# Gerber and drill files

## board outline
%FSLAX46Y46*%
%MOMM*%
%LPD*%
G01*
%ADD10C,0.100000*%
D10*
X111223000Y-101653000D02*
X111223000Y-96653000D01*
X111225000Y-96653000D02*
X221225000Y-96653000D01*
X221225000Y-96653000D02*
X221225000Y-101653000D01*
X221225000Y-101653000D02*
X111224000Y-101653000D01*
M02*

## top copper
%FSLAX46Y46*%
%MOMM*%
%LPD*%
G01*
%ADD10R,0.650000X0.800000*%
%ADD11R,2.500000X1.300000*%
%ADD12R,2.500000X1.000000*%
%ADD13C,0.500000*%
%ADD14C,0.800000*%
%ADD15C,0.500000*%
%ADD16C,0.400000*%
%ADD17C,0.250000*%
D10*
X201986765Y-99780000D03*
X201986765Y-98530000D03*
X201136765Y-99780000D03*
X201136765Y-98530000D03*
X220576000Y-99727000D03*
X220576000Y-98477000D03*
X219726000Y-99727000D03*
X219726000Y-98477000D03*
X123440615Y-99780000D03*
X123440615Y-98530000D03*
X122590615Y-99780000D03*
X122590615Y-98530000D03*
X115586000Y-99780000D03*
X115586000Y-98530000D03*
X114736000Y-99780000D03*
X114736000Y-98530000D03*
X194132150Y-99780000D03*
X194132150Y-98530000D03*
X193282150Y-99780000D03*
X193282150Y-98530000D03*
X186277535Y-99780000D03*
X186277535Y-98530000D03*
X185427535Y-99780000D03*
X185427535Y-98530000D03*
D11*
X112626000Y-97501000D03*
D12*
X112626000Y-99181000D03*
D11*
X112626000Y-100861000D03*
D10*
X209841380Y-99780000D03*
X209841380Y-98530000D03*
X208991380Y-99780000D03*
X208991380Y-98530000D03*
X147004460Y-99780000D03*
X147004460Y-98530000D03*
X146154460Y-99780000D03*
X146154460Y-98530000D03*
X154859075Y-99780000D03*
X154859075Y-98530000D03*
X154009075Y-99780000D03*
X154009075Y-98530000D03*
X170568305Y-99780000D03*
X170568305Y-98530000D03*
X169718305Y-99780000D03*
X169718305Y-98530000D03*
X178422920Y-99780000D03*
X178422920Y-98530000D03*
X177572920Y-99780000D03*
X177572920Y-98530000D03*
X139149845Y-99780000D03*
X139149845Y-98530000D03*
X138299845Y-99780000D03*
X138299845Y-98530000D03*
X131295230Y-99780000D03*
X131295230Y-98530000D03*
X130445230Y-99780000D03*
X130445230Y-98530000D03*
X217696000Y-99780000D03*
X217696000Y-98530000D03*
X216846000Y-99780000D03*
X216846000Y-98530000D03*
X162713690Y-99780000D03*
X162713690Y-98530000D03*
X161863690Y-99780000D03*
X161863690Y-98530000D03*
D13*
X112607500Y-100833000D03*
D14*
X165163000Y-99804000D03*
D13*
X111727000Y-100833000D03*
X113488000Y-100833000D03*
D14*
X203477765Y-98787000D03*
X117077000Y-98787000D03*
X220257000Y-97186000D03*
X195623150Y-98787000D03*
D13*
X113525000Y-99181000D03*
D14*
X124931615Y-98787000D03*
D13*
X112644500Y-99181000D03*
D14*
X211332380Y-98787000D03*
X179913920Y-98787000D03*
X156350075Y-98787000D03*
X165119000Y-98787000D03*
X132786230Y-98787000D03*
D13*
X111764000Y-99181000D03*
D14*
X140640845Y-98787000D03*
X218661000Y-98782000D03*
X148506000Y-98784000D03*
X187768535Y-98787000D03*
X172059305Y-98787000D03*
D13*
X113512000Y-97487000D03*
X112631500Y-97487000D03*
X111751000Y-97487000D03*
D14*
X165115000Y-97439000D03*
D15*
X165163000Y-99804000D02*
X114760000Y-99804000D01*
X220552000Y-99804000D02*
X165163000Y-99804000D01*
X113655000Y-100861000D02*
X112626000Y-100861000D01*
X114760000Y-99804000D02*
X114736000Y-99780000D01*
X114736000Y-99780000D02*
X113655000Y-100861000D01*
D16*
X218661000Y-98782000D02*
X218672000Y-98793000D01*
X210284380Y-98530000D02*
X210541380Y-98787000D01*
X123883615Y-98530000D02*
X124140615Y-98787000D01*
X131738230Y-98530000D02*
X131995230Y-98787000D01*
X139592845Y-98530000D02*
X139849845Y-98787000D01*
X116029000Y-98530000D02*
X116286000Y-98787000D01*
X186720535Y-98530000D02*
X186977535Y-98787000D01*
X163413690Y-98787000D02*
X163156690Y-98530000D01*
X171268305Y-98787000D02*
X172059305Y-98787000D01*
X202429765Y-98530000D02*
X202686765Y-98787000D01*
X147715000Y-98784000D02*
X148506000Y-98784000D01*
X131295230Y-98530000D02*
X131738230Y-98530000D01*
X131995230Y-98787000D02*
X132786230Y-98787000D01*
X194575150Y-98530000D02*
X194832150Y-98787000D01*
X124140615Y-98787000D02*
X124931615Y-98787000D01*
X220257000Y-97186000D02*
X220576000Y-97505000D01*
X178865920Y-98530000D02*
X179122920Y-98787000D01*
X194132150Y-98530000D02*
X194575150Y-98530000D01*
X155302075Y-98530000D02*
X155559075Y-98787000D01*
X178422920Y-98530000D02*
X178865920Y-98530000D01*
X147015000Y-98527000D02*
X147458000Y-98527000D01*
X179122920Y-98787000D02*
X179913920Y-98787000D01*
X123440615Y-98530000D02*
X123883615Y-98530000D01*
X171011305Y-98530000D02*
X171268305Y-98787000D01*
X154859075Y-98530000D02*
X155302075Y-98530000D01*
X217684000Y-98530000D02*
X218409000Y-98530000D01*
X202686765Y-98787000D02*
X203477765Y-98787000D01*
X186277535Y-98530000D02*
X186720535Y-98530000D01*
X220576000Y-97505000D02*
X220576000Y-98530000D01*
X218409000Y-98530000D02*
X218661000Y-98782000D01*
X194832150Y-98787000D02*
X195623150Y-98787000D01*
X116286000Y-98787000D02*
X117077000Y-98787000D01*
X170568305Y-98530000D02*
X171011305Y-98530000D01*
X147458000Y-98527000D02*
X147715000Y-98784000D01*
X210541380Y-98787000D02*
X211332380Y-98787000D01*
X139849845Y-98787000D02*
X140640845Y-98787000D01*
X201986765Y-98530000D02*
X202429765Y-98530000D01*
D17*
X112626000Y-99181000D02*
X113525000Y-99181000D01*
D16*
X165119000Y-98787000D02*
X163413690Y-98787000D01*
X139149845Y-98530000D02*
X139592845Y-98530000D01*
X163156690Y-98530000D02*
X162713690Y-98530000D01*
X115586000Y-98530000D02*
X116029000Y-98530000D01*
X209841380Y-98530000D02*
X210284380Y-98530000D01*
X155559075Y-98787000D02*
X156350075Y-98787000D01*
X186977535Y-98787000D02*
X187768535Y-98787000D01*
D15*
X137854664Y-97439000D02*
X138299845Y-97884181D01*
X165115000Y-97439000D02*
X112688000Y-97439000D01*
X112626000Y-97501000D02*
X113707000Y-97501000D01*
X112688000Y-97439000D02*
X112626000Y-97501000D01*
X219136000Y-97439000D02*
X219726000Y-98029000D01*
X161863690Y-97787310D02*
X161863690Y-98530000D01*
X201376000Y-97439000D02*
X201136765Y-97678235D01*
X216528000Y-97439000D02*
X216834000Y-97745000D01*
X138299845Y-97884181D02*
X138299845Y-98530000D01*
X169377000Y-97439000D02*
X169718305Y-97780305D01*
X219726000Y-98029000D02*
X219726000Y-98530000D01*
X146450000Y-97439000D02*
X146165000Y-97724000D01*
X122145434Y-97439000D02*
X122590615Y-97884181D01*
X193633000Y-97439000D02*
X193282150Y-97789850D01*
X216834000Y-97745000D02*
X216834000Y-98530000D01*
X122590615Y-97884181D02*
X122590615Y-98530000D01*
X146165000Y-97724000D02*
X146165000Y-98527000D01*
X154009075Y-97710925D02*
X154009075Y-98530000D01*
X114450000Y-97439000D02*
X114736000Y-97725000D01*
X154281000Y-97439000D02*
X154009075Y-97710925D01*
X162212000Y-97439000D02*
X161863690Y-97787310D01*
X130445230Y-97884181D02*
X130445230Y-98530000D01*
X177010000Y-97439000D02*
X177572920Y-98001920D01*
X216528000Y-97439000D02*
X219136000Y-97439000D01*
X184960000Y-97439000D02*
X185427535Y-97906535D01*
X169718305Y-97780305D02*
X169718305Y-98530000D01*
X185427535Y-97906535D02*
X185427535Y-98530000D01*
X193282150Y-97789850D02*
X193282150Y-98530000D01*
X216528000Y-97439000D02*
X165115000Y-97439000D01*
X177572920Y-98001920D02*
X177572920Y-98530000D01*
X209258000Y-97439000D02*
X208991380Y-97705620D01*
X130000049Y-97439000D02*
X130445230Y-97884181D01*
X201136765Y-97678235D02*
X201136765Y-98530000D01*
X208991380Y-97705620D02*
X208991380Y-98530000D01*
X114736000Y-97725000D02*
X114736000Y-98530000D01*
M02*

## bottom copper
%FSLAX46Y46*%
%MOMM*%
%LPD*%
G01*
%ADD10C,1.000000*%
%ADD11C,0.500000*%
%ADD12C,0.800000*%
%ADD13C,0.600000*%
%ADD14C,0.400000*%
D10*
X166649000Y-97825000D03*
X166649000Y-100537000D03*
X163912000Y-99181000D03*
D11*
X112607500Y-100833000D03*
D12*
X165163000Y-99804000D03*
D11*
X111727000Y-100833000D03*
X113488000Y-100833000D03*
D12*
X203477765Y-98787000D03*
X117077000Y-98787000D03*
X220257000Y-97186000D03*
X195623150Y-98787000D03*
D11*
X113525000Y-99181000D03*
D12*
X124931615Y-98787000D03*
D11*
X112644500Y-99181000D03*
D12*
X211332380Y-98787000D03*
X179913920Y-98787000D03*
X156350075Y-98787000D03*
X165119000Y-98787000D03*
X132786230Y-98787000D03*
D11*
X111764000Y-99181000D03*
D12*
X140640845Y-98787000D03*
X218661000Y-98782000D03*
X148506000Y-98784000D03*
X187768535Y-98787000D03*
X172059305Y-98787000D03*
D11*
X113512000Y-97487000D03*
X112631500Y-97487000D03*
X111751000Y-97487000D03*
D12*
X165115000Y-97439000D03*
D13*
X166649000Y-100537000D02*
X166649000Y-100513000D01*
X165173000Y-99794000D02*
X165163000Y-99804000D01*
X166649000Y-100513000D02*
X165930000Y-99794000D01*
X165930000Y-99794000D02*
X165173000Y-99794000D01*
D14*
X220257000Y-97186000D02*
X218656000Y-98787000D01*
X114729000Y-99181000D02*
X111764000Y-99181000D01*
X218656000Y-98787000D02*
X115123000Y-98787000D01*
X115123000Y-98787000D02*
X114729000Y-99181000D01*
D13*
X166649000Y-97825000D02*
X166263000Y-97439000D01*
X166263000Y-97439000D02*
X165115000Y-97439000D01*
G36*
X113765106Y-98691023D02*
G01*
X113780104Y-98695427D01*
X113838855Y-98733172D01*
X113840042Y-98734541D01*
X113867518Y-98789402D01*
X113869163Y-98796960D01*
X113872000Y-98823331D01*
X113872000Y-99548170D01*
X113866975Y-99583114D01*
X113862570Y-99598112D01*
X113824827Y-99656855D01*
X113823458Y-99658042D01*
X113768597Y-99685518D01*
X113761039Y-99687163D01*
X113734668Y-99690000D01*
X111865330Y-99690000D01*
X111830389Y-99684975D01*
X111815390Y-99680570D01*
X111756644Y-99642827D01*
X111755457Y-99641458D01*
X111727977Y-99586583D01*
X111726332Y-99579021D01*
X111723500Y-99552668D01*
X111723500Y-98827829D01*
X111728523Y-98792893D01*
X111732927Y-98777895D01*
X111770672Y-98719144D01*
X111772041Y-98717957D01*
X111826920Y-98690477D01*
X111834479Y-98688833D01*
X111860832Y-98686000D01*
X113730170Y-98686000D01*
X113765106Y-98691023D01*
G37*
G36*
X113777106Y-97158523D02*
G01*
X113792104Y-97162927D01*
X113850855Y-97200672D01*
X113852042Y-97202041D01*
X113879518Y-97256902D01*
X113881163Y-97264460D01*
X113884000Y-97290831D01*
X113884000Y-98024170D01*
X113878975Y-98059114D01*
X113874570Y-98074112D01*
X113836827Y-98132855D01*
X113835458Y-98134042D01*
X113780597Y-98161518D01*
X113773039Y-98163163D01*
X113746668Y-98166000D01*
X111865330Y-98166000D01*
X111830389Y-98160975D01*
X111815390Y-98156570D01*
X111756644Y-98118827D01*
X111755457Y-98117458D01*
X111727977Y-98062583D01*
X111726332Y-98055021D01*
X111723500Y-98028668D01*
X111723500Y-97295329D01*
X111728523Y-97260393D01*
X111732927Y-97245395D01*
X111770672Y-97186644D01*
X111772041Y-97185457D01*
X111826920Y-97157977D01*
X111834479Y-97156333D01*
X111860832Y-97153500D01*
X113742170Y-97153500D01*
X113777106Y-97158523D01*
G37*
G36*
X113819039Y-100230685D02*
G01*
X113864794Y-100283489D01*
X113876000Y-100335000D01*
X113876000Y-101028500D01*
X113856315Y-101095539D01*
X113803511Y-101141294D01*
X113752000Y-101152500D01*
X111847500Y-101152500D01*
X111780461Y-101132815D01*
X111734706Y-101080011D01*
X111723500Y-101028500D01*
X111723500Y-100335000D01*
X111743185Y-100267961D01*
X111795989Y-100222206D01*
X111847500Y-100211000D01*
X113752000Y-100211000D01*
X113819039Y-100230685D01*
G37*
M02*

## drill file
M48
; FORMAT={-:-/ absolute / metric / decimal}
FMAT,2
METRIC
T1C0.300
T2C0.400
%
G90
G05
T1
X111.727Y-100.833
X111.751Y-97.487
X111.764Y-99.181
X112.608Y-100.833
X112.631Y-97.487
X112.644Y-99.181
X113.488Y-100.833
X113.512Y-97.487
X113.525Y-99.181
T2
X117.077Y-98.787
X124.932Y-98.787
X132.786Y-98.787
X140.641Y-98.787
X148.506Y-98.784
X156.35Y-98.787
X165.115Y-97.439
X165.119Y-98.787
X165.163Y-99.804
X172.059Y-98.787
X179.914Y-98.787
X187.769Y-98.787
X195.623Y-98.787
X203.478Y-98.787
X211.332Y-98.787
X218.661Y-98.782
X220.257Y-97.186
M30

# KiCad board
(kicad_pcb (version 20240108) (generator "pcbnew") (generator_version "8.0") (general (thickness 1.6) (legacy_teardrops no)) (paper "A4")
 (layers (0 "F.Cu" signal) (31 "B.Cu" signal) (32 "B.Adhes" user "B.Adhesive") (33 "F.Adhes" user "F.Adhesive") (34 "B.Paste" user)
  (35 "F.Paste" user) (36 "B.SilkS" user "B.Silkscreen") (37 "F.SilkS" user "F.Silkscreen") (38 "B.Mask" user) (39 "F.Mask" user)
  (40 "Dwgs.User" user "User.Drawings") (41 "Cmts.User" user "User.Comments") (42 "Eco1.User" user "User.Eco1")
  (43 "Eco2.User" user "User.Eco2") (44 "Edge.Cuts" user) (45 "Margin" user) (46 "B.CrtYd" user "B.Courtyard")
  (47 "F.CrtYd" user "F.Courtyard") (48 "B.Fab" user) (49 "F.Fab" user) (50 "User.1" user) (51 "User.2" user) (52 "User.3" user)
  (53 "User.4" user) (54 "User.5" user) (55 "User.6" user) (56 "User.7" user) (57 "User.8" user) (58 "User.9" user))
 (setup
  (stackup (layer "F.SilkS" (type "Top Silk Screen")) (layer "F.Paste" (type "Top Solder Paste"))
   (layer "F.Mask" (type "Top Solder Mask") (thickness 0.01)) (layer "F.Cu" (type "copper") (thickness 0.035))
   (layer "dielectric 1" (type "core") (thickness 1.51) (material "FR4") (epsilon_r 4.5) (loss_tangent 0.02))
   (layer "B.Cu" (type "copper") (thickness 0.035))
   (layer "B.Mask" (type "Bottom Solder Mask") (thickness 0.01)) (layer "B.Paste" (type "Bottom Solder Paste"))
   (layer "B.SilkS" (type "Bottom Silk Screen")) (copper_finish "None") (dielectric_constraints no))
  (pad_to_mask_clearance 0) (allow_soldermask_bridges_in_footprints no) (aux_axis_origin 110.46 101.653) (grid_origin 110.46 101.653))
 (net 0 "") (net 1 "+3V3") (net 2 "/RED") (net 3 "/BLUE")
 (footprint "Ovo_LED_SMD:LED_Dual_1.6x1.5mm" (layer "F.Cu") (at 201.561765 99.155 90)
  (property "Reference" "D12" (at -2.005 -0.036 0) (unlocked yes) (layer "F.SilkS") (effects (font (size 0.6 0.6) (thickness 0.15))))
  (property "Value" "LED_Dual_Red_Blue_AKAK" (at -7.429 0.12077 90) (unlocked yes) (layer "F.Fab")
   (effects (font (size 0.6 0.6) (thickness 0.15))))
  (pad "1" smd rect (at -0.625 0.425 90) (size 0.8 0.65) (layers "F.Cu" "F.Paste" "F.Mask") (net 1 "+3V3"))
  (pad "2" smd rect (at 0.625 0.425 90) (size 0.8 0.65) (layers "F.Cu" "F.Paste" "F.Mask") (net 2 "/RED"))
  (pad "3" smd rect (at -0.625 -0.425 90) (size 0.8 0.65) (layers "F.Cu" "F.Paste" "F.Mask") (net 1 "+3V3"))
  (pad "4" smd rect (at 0.625 -0.425 90) (size 0.8 0.65) (layers "F.Cu" "F.Paste" "F.Mask") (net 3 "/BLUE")))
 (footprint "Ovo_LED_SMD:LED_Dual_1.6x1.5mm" (layer "F.Cu") (at 220.151 99.102 90)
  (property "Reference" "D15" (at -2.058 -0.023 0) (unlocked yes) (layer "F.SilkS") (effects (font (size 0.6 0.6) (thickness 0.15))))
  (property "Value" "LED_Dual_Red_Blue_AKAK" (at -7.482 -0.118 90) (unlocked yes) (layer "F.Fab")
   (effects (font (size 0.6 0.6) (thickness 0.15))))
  (pad "1" smd rect (at -0.625 0.425 90) (size 0.8 0.65) (layers "F.Cu" "F.Paste" "F.Mask") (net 1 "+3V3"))
  (pad "2" smd rect (at 0.625 0.425 90) (size 0.8 0.65) (layers "F.Cu" "F.Paste" "F.Mask") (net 2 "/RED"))
  (pad "3" smd rect (at -0.625 -0.425 90) (size 0.8 0.65) (layers "F.Cu" "F.Paste" "F.Mask") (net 1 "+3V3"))
  (pad "4" smd rect (at 0.625 -0.425 90) (size 0.8 0.65) (layers "F.Cu" "F.Paste" "F.Mask") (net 3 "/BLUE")))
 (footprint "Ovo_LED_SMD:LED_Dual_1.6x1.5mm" (layer "F.Cu") (at 123.015615 99.155 90)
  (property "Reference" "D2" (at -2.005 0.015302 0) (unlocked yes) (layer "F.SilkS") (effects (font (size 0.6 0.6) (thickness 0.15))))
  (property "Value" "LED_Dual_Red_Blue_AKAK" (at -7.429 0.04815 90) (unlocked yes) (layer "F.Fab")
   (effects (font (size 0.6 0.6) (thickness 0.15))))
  (pad "1" smd rect (at -0.625 0.425 90) (size 0.8 0.65) (layers "F.Cu" "F.Paste" "F.Mask") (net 1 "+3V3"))
  (pad "2" smd rect (at 0.625 0.425 90) (size 0.8 0.65) (layers "F.Cu" "F.Paste" "F.Mask") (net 2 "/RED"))
  (pad "3" smd rect (at -0.625 -0.425 90) (size 0.8 0.65) (layers "F.Cu" "F.Paste" "F.Mask") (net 1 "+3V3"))
  (pad "4" smd rect (at 0.625 -0.425 90) (size 0.8 0.65) (layers "F.Cu" "F.Paste" "F.Mask") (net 3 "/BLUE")))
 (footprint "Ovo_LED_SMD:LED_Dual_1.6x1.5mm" (layer "F.Cu") (at 115.161 99.155 90)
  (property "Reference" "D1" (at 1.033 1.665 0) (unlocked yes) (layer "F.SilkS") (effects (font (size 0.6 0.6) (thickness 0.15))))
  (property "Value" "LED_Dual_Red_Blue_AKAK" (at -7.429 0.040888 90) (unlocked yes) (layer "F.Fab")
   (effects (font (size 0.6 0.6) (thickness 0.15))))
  (pad "1" smd rect (at -0.625 0.425 90) (size 0.8 0.65) (layers "F.Cu" "F.Paste" "F.Mask") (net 1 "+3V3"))
  (pad "2" smd rect (at 0.625 0.425 90) (size 0.8 0.65) (layers "F.Cu" "F.Paste" "F.Mask") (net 2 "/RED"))
  (pad "3" smd rect (at -0.625 -0.425 90) (size 0.8 0.65) (layers "F.Cu" "F.Paste" "F.Mask") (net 1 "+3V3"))
  (pad "4" smd rect (at 0.625 -0.425 90) (size 0.8 0.65) (layers "F.Cu" "F.Paste" "F.Mask") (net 3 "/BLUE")))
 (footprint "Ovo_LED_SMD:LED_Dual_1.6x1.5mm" (layer "F.Cu") (at 193.70715 99.155 90)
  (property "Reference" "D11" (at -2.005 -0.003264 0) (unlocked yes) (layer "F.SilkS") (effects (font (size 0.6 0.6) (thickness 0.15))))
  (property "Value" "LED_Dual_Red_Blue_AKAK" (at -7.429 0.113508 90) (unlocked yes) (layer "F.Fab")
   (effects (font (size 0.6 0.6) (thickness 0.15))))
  (pad "1" smd rect (at -0.625 0.425 90) (size 0.8 0.65) (layers "F.Cu" "F.Paste" "F.Mask") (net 1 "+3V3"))
  (pad "2" smd rect (at 0.625 0.425 90) (size 0.8 0.65) (layers "F.Cu" "F.Paste" "F.Mask") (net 2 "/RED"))
  (pad "3" smd rect (at -0.625 -0.425 90) (size 0.8 0.65) (layers "F.Cu" "F.Paste" "F.Mask") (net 1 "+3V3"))
  (pad "4" smd rect (at 0.625 -0.425 90) (size 0.8 0.65) (layers "F.Cu" "F.Paste" "F.Mask") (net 3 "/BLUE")))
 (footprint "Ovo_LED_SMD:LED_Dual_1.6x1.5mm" (layer "F.Cu") (at 185.852535 99.155 90)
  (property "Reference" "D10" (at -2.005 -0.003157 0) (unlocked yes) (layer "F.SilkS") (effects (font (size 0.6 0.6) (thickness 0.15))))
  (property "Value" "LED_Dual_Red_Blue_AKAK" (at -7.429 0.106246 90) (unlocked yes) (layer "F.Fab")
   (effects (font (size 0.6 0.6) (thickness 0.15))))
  (pad "1" smd rect (at -0.625 0.425 90) (size 0.8 0.65) (layers "F.Cu" "F.Paste" "F.Mask") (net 1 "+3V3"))
  (pad "2" smd rect (at 0.625 0.425 90) (size 0.8 0.65) (layers "F.Cu" "F.Paste" "F.Mask") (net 2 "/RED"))
  (pad "3" smd rect (at -0.625 -0.425 90) (size 0.8 0.65) (layers "F.Cu" "F.Paste" "F.Mask") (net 1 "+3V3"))
  (pad "4" smd rect (at 0.625 -0.425 90) (size 0.8 0.65) (layers "F.Cu" "F.Paste" "F.Mask") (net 3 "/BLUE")))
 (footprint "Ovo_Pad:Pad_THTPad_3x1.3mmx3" (layer "F.Cu") (at 112.666 97.511)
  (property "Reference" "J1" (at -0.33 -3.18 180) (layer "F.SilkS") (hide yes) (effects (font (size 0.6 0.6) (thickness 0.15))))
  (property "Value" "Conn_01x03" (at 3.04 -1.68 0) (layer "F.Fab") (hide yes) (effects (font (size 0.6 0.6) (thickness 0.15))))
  (pad "1" smd rect (at -0.04 -0.01 180) (size 2.5 1.3) (layers "F.Cu" "F.Paste" "F.Mask") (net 3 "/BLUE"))
  (pad "2" smd rect (at -0.04 1.67 180) (size 2.5 1) (layers "F.Cu" "F.Paste" "F.Mask") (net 2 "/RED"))
  (pad "3" smd rect (at -0.04 3.35 180) (size 2.5 1.3) (layers "F.Cu" "F.Paste" "F.Mask") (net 1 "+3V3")))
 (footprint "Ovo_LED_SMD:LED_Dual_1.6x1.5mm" (layer "F.Cu") (at 209.41638 99.155 90)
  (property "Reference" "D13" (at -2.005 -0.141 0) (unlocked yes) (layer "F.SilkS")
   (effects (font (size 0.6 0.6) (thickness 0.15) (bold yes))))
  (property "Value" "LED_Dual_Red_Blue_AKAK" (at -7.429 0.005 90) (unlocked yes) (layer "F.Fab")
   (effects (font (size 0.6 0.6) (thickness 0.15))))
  (pad "1" smd rect (at -0.625 0.425 90) (size 0.8 0.65) (layers "F.Cu" "F.Paste" "F.Mask") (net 1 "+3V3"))
  (pad "2" smd rect (at 0.625 0.425 90) (size 0.8 0.65) (layers "F.Cu" "F.Paste" "F.Mask") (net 2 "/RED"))
  (pad "3" smd rect (at -0.625 -0.425 90) (size 0.8 0.65) (layers "F.Cu" "F.Paste" "F.Mask") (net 1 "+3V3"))
  (pad "4" smd rect (at 0.625 -0.425 90) (size 0.8 0.65) (layers "F.Cu" "F.Paste" "F.Mask") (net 3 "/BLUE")))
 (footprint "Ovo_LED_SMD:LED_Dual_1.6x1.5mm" (layer "F.Cu") (at 146.57946 99.155 90)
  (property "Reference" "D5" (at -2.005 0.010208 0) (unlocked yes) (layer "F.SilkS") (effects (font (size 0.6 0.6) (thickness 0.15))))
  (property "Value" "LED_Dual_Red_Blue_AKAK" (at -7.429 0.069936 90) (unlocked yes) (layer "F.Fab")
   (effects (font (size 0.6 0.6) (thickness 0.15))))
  (pad "1" smd rect (at -0.625 0.425 90) (size 0.8 0.65) (layers "F.Cu" "F.Paste" "F.Mask") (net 1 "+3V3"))
  (pad "2" smd rect (at 0.625 0.425 90) (size 0.8 0.65) (layers "F.Cu" "F.Paste" "F.Mask") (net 2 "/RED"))
  (pad "3" smd rect (at -0.625 -0.425 90) (size 0.8 0.65) (layers "F.Cu" "F.Paste" "F.Mask") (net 1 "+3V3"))
  (pad "4" smd rect (at 0.625 -0.425 90) (size 0.8 0.65) (layers "F.Cu" "F.Paste" "F.Mask") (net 3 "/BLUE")))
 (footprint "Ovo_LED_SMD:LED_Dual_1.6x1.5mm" (layer "F.Cu") (at 154.434075 99.155 90)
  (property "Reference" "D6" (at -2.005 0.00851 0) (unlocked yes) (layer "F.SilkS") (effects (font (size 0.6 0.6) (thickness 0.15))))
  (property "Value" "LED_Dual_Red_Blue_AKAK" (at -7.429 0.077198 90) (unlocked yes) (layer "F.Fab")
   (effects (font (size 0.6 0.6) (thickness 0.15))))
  (pad "1" smd rect (at -0.625 0.425 90) (size 0.8 0.65) (layers "F.Cu" "F.Paste" "F.Mask") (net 1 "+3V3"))
  (pad "2" smd rect (at 0.625 0.425 90) (size 0.8 0.65) (layers "F.Cu" "F.Paste" "F.Mask") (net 2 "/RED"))
  (pad "3" smd rect (at -0.625 -0.425 90) (size 0.8 0.65) (layers "F.Cu" "F.Paste" "F.Mask") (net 1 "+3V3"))
  (pad "4" smd rect (at 0.625 -0.425 90) (size 0.8 0.65) (layers "F.Cu" "F.Paste" "F.Mask") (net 3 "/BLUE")))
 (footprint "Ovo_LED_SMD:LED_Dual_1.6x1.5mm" (layer "F.Cu") (at 170.143305 99.155 90)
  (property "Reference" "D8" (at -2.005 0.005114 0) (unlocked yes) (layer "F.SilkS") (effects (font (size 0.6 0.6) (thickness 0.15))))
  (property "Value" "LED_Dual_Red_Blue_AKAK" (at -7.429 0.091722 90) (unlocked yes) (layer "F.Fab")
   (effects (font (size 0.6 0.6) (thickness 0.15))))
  (pad "1" smd rect (at -0.625 0.425 90) (size 0.8 0.65) (layers "F.Cu" "F.Paste" "F.Mask") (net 1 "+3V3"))
  (pad "2" smd rect (at 0.625 0.425 90) (size 0.8 0.65) (layers "F.Cu" "F.Paste" "F.Mask") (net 2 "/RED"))
  (pad "3" smd rect (at -0.625 -0.425 90) (size 0.8 0.65) (layers "F.Cu" "F.Paste" "F.Mask") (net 1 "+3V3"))
  (pad "4" smd rect (at 0.625 -0.425 90) (size 0.8 0.65) (layers "F.Cu" "F.Paste" "F.Mask") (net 3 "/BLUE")))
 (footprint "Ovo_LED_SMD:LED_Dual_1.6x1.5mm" (layer "F.Cu") (at 177.99792 99.155 90)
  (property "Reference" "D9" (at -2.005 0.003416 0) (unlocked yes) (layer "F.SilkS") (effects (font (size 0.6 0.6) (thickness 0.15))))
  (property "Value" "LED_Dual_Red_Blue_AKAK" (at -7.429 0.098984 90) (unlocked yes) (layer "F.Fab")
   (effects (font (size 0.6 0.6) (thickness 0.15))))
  (pad "1" smd rect (at -0.625 0.425 90) (size 0.8 0.65) (layers "F.Cu" "F.Paste" "F.Mask") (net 1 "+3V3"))
  (pad "2" smd rect (at 0.625 0.425 90) (size 0.8 0.65) (layers "F.Cu" "F.Paste" "F.Mask") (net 2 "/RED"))
  (pad "3" smd rect (at -0.625 -0.425 90) (size 0.8 0.65) (layers "F.Cu" "F.Paste" "F.Mask") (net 1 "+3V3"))
  (pad "4" smd rect (at 0.625 -0.425 90) (size 0.8 0.65) (layers "F.Cu" "F.Paste" "F.Mask") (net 3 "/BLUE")))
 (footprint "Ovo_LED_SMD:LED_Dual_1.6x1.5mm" (layer "F.Cu") (at 138.724845 99.155 90)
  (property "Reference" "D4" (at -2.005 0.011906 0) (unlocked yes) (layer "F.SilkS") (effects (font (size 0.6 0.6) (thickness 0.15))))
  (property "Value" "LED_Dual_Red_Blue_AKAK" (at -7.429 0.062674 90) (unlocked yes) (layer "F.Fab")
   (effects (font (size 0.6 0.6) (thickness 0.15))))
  (pad "1" smd rect (at -0.625 0.425 90) (size 0.8 0.65) (layers "F.Cu" "F.Paste" "F.Mask") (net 1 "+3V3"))
  (pad "2" smd rect (at 0.625 0.425 90) (size 0.8 0.65) (layers "F.Cu" "F.Paste" "F.Mask") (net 2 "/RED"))
  (pad "3" smd rect (at -0.625 -0.425 90) (size 0.8 0.65) (layers "F.Cu" "F.Paste" "F.Mask") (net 1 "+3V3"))
  (pad "4" smd rect (at 0.625 -0.425 90) (size 0.8 0.65) (layers "F.Cu" "F.Paste" "F.Mask") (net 3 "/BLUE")))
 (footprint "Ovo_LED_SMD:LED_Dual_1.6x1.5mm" (layer "F.Cu") (at 130.87023 99.155 90)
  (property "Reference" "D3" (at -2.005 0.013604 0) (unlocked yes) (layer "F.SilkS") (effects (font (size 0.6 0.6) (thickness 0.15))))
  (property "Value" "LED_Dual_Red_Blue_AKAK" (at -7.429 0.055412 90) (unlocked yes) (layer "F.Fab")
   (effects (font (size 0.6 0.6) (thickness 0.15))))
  (pad "1" smd rect (at -0.625 0.425 90) (size 0.8 0.65) (layers "F.Cu" "F.Paste" "F.Mask") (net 1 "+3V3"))
  (pad "2" smd rect (at 0.625 0.425 90) (size 0.8 0.65) (layers "F.Cu" "F.Paste" "F.Mask") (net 2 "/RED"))
  (pad "3" smd rect (at -0.625 -0.425 90) (size 0.8 0.65) (layers "F.Cu" "F.Paste" "F.Mask") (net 1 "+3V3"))
  (pad "4" smd rect (at 0.625 -0.425 90) (size 0.8 0.65) (layers "F.Cu" "F.Paste" "F.Mask") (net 3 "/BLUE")))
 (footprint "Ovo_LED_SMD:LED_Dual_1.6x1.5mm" (layer "F.Cu") (at 217.271 99.155 90)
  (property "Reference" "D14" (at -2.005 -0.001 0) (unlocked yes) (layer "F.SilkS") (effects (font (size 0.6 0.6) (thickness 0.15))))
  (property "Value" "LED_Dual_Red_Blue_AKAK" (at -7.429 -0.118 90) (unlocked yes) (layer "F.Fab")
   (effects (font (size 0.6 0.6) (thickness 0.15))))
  (pad "1" smd rect (at -0.625 0.425 90) (size 0.8 0.65) (layers "F.Cu" "F.Paste" "F.Mask") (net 1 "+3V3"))
  (pad "2" smd rect (at 0.625 0.425 90) (size 0.8 0.65) (layers "F.Cu" "F.Paste" "F.Mask") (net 2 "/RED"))
  (pad "3" smd rect (at -0.625 -0.425 90) (size 0.8 0.65) (layers "F.Cu" "F.Paste" "F.Mask") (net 1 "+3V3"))
  (pad "4" smd rect (at 0.625 -0.425 90) (size 0.8 0.65) (layers "F.Cu" "F.Paste" "F.Mask") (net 3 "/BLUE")))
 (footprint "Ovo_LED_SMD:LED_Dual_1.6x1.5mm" (layer "F.Cu") (at 162.28869 99.155 90)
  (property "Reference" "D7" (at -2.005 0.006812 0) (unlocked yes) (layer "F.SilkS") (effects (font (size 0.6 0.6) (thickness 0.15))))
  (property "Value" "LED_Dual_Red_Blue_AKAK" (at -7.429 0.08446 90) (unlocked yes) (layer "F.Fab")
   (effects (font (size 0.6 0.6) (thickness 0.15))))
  (pad "1" smd rect (at -0.625 0.425 90) (size 0.8 0.65) (layers "F.Cu" "F.Paste" "F.Mask") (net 1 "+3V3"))
  (pad "2" smd rect (at 0.625 0.425 90) (size 0.8 0.65) (layers "F.Cu" "F.Paste" "F.Mask") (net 2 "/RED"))
  (pad "3" smd rect (at -0.625 -0.425 90) (size 0.8 0.65) (layers "F.Cu" "F.Paste" "F.Mask") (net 1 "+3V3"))
  (pad "4" smd rect (at 0.625 -0.425 90) (size 0.8 0.65) (layers "F.Cu" "F.Paste" "F.Mask") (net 3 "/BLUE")))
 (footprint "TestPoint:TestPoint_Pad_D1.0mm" (layer "B.Cu") (at 166.649 97.825 180)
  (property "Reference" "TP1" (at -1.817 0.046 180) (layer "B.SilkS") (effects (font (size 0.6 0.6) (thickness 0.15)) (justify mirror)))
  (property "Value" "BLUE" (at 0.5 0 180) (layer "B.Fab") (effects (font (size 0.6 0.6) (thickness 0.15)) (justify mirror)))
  (pad "1" smd circle (at 0 0 180) (size 1 1) (layers "B.Cu" "B.Mask") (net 3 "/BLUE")))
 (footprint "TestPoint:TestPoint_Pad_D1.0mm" (layer "B.Cu") (at 166.649 100.537 180)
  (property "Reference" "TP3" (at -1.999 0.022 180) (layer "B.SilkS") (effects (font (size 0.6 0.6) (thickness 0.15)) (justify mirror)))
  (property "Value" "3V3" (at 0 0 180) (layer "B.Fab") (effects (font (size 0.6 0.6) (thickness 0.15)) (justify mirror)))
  (pad "1" smd circle (at 0 0 180) (size 1 1) (layers "B.Cu" "B.Mask") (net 1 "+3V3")))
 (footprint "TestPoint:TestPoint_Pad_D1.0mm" (layer "B.Cu") (at 163.912 99.181 180)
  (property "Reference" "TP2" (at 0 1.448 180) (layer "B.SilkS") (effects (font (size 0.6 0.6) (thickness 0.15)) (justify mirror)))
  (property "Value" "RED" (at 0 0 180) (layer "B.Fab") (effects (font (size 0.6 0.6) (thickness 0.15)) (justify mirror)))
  (pad "1" smd circle (at 0 0 180) (size 1 1) (layers "B.Cu" "B.Mask") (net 2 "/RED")))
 (gr_line (start 111.223 101.653) (end 111.223 96.653) (stroke (width 0.1) (type default)) (layer "Edge.Cuts"))
 (gr_line (start 111.225 96.653) (end 221.225 96.653) (stroke (width 0.1) (type default)) (layer "Edge.Cuts"))
 (gr_line (start 221.225 96.653) (end 221.225 101.653) (stroke (width 0.1) (type default)) (layer "Edge.Cuts"))
 (gr_line (start 221.225 101.653) (end 111.224 101.653) (stroke (width 0.1) (type default)) (layer "Edge.Cuts"))
 (segment (start 165.163 99.804) (end 114.76 99.804) (width 0.5) (layer "F.Cu") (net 1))
 (segment (start 220.552 99.804) (end 165.163 99.804) (width 0.5) (layer "F.Cu") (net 1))
 (segment (start 113.655 100.861) (end 112.626 100.861) (width 0.5) (layer "F.Cu") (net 1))
 (segment (start 114.76 99.804) (end 114.736 99.78) (width 0.5) (layer "F.Cu") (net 1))
 (segment (start 114.736 99.78) (end 113.655 100.861) (width 0.5) (layer "F.Cu") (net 1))
 (via (at 112.6075 100.833) (size 0.5) (drill 0.3) (layers "F.Cu" "B.Cu") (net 1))
 (via (at 165.163 99.804) (size 0.8) (drill 0.4) (layers "F.Cu" "B.Cu") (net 1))
 (via (at 111.727 100.833) (size 0.5) (drill 0.3) (layers "F.Cu" "B.Cu") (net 1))
 (via (at 113.488 100.833) (size 0.5) (drill 0.3) (layers "F.Cu" "B.Cu") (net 1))
 (segment (start 166.649 100.537) (end 166.649 100.513) (width 0.6) (layer "B.Cu") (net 1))
 (segment (start 165.173 99.794) (end 165.163 99.804) (width 0.6) (layer "B.Cu") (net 1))
 (segment (start 166.649 100.513) (end 165.93 99.794) (width 0.6) (layer "B.Cu") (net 1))
 (segment (start 165.93 99.794) (end 165.173 99.794) (width 0.6) (layer "B.Cu") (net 1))
 (segment (start 218.661 98.782) (end 218.672 98.793) (width 0.4) (layer "F.Cu") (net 2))
 (segment (start 210.28438 98.53) (end 210.54138 98.787) (width 0.4) (layer "F.Cu") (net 2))
 (segment (start 123.883615 98.53) (end 124.140615 98.787) (width 0.4) (layer "F.Cu") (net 2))
 (segment (start 131.73823 98.53) (end 131.99523 98.787) (width 0.4) (layer "F.Cu") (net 2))
 (segment (start 139.592845 98.53) (end 139.849845 98.787) (width 0.4) (layer "F.Cu") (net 2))
 (segment (start 116.029 98.53) (end 116.286 98.787) (width 0.4) (layer "F.Cu") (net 2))
 (segment (start 186.720535 98.53) (end 186.977535 98.787) (width 0.4) (layer "F.Cu") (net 2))
 (segment (start 163.41369 98.787) (end 163.15669 98.53) (width 0.4) (layer "F.Cu") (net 2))
 (segment (start 171.268305 98.787) (end 172.059305 98.787) (width 0.4) (layer "F.Cu") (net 2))
 (segment (start 202.429765 98.53) (end 202.686765 98.787) (width 0.4) (layer "F.Cu") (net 2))
 (segment (start 147.715 98.784) (end 148.506 98.784) (width 0.4) (layer "F.Cu") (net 2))
 (segment (start 131.29523 98.53) (end 131.73823 98.53) (width 0.4) (layer "F.Cu") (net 2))
 (segment (start 131.99523 98.787) (end 132.78623 98.787) (width 0.4) (layer "F.Cu") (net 2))
 (segment (start 194.57515 98.53) (end 194.83215 98.787) (width 0.4) (layer "F.Cu") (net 2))
 (segment (start 124.140615 98.787) (end 124.931615 98.787) (width 0.4) (layer "F.Cu") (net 2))
 (segment (start 220.257 97.186) (end 220.576 97.505) (width 0.4) (layer "F.Cu") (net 2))
 (segment (start 178.86592 98.53) (end 179.12292 98.787) (width 0.4) (layer "F.Cu") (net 2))
 (segment (start 194.13215 98.53) (end 194.57515 98.53) (width 0.4) (layer "F.Cu") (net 2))
 (segment (start 155.302075 98.53) (end 155.559075 98.787) (width 0.4) (layer "F.Cu") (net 2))
 (segment (start 178.42292 98.53) (end 178.86592 98.53) (width 0.4) (layer "F.Cu") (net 2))
 (segment (start 147.015 98.527) (end 147.458 98.527) (width 0.4) (layer "F.Cu") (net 2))
 (segment (start 179.12292 98.787) (end 179.91392 98.787) (width 0.4) (layer "F.Cu") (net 2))
 (segment (start 123.440615 98.53) (end 123.883615 98.53) (width 0.4) (layer "F.Cu") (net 2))
 (segment (start 171.011305 98.53) (end 171.268305 98.787) (width 0.4) (layer "F.Cu") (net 2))
 (segment (start 154.859075 98.53) (end 155.302075 98.53) (width 0.4) (layer "F.Cu") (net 2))
 (segment (start 217.684 98.53) (end 218.409 98.53) (width 0.4) (layer "F.Cu") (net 2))
 (segment (start 202.686765 98.787) (end 203.477765 98.787) (width 0.4) (layer "F.Cu") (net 2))
 (segment (start 186.277535 98.53) (end 186.720535 98.53) (width 0.4) (layer "F.Cu") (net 2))
 (segment (start 220.576 97.505) (end 220.576 98.53) (width 0.4) (layer "F.Cu") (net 2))
 (segment (start 218.409 98.53) (end 218.661 98.782) (width 0.4) (layer "F.Cu") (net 2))
 (segment (start 194.83215 98.787) (end 195.62315 98.787) (width 0.4) (layer "F.Cu") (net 2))
 (segment (start 116.286 98.787) (end 117.077 98.787) (width 0.4) (layer "F.Cu") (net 2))
 (segment (start 170.568305 98.53) (end 171.011305 98.53) (width 0.4) (layer "F.Cu") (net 2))
 (segment (start 147.458 98.527) (end 147.715 98.784) (width 0.4) (layer "F.Cu") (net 2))
 (segment (start 210.54138 98.787) (end 211.33238 98.787) (width 0.4) (layer "F.Cu") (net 2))
 (segment (start 139.849845 98.787) (end 140.640845 98.787) (width 0.4) (layer "F.Cu") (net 2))
 (segment (start 201.986765 98.53) (end 202.429765 98.53) (width 0.4) (layer "F.Cu") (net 2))
 (segment (start 112.626 99.181) (end 113.525 99.181) (width 0.25) (layer "F.Cu") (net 2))
 (segment (start 165.119 98.787) (end 163.41369 98.787) (width 0.4) (layer "F.Cu") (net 2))
 (segment (start 139.149845 98.53) (end 139.592845 98.53) (width 0.4) (layer "F.Cu") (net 2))
 (segment (start 163.15669 98.53) (end 162.71369 98.53) (width 0.4) (layer "F.Cu") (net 2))
 (segment (start 115.586 98.53) (end 116.029 98.53) (width 0.4) (layer "F.Cu") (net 2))
 (segment (start 209.84138 98.53) (end 210.28438 98.53) (width 0.4) (layer "F.Cu") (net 2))
 (segment (start 155.559075 98.787) (end 156.350075 98.787) (width 0.4) (layer "F.Cu") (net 2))
 (segment (start 186.977535 98.787) (end 187.768535 98.787) (width 0.4) (layer "F.Cu") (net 2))
 (via (at 203.477765 98.787) (size 0.8) (drill 0.4) (layers "F.Cu" "B.Cu") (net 2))
 (via (at 117.077 98.787) (size 0.8) (drill 0.4) (layers "F.Cu" "B.Cu") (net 2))
 (via (at 220.257 97.186) (size 0.8) (drill 0.4) (layers "F.Cu" "B.Cu") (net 2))
 (via (at 195.62315 98.787) (size 0.8) (drill 0.4) (layers "F.Cu" "B.Cu") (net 2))
 (via (at 113.525 99.181) (size 0.5) (drill 0.3) (layers "F.Cu" "B.Cu") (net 2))
 (via (at 124.931615 98.787) (size 0.8) (drill 0.4) (layers "F.Cu" "B.Cu") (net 2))
 (via (at 112.6445 99.181) (size 0.5) (drill 0.3) (layers "F.Cu" "B.Cu") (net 2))
 (via (at 211.33238 98.787) (size 0.8) (drill 0.4) (layers "F.Cu" "B.Cu") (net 2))
 (via (at 179.91392 98.787) (size 0.8) (drill 0.4) (layers "F.Cu" "B.Cu") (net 2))
 (via (at 156.350075 98.787) (size 0.8) (drill 0.4) (layers "F.Cu" "B.Cu") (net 2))
 (via (at 165.119 98.787) (size 0.8) (drill 0.4) (layers "F.Cu" "B.Cu") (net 2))
 (via (at 132.78623 98.787) (size 0.8) (drill 0.4) (layers "F.Cu" "B.Cu") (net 2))
 (via (at 111.764 99.181) (size 0.5) (drill 0.3) (layers "F.Cu" "B.Cu") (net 2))
 (via (at 140.640845 98.787) (size 0.8) (drill 0.4) (layers "F.Cu" "B.Cu") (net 2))
 (via (at 218.661 98.782) (size 0.8) (drill 0.4) (layers "F.Cu" "B.Cu") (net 2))
 (via (at 148.506 98.784) (size 0.8) (drill 0.4) (layers "F.Cu" "B.Cu") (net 2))
 (via (at 187.768535 98.787) (size 0.8) (drill 0.4) (layers "F.Cu" "B.Cu") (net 2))
 (via (at 172.059305 98.787) (size 0.8) (drill 0.4) (layers "F.Cu" "B.Cu") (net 2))
 (segment (start 220.257 97.186) (end 218.656 98.787) (width 0.4) (layer "B.Cu") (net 2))
 (segment (start 114.729 99.181) (end 111.764 99.181) (width 0.4) (layer "B.Cu") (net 2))
 (segment (start 218.656 98.787) (end 115.123 98.787) (width 0.4) (layer "B.Cu") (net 2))
 (segment (start 115.123 98.787) (end 114.729 99.181) (width 0.4) (layer "B.Cu") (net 2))
 (segment (start 137.854664 97.439) (end 138.299845 97.884181) (width 0.5) (layer "F.Cu") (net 3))
 (segment (start 165.115 97.439) (end 112.688 97.439) (width 0.5) (layer "F.Cu") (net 3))
 (segment (start 112.626 97.501) (end 113.707 97.501) (width 0.5) (layer "F.Cu") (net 3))
 (segment (start 112.688 97.439) (end 112.626 97.501) (width 0.5) (layer "F.Cu") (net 3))
 (segment (start 219.136 97.439) (end 219.726 98.029) (width 0.5) (layer "F.Cu") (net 3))
 (segment (start 161.86369 97.78731) (end 161.86369 98.53) (width 0.5) (layer "F.Cu") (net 3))
 (segment (start 201.376 97.439) (end 201.136765 97.678235) (width 0.5) (layer "F.Cu") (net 3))
 (segment (start 216.528 97.439) (end 216.834 97.745) (width 0.5) (layer "F.Cu") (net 3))
 (segment (start 138.299845 97.884181) (end 138.299845 98.53) (width 0.5) (layer "F.Cu") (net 3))
 (segment (start 169.377 97.439) (end 169.718305 97.780305) (width 0.5) (layer "F.Cu") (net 3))
 (segment (start 219.726 98.029) (end 219.726 98.53) (width 0.5) (layer "F.Cu") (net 3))
 (segment (start 146.45 97.439) (end 146.165 97.724) (width 0.5) (layer "F.Cu") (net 3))
 (segment (start 122.145434 97.439) (end 122.590615 97.884181) (width 0.5) (layer "F.Cu") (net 3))
 (segment (start 193.633 97.439) (end 193.28215 97.78985) (width 0.5) (layer "F.Cu") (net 3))
 (segment (start 216.834 97.745) (end 216.834 98.53) (width 0.5) (layer "F.Cu") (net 3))
 (segment (start 122.590615 97.884181) (end 122.590615 98.53) (width 0.5) (layer "F.Cu") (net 3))
 (segment (start 146.165 97.724) (end 146.165 98.527) (width 0.5) (layer "F.Cu") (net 3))
 (segment (start 154.009075 97.710925) (end 154.009075 98.53) (width 0.5) (layer "F.Cu") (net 3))
 (segment (start 114.45 97.439) (end 114.736 97.725) (width 0.5) (layer "F.Cu") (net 3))
 (segment (start 154.281 97.439) (end 154.009075 97.710925) (width 0.5) (layer "F.Cu") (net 3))
 (segment (start 162.212 97.439) (end 161.86369 97.78731) (width 0.5) (layer "F.Cu") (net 3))
 (segment (start 130.44523 97.884181) (end 130.44523 98.53) (width 0.5) (layer "F.Cu") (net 3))
 (segment (start 177.01 97.439) (end 177.57292 98.00192) (width 0.5) (layer "F.Cu") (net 3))
 (segment (start 216.528 97.439) (end 219.136 97.439) (width 0.5) (layer "F.Cu") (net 3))
 (segment (start 184.96 97.439) (end 185.427535 97.906535) (width 0.5) (layer "F.Cu") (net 3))
 (segment (start 169.718305 97.780305) (end 169.718305 98.53) (width 0.5) (layer "F.Cu") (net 3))
 (segment (start 185.427535 97.906535) (end 185.427535 98.53) (width 0.5) (layer "F.Cu") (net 3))
 (segment (start 193.28215 97.78985) (end 193.28215 98.53) (width 0.5) (layer "F.Cu") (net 3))
 (segment (start 216.528 97.439) (end 165.115 97.439) (width 0.5) (layer "F.Cu") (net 3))
 (segment (start 177.57292 98.00192) (end 177.57292 98.53) (width 0.5) (layer "F.Cu") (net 3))
 (segment (start 209.258 97.439) (end 208.99138 97.70562) (width 0.5) (layer "F.Cu") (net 3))
 (segment (start 130.000049 97.439) (end 130.44523 97.884181) (width 0.5) (layer "F.Cu") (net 3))
 (segment (start 201.136765 97.678235) (end 201.136765 98.53) (width 0.5) (layer "F.Cu") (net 3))
 (segment (start 208.99138 97.70562) (end 208.99138 98.53) (width 0.5) (layer "F.Cu") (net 3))
 (segment (start 114.736 97.725) (end 114.736 98.53) (width 0.5) (layer "F.Cu") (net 3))
 (via (at 113.512 97.487) (size 0.5) (drill 0.3) (layers "F.Cu" "B.Cu") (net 3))
 (via (at 112.6315 97.487) (size 0.5) (drill 0.3) (layers "F.Cu" "B.Cu") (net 3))
 (via (at 111.751 97.487) (size 0.5) (drill 0.3) (layers "F.Cu" "B.Cu") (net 3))
 (via (at 165.115 97.439) (size 0.8) (drill 0.4) (layers "F.Cu" "B.Cu") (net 3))
 (segment (start 166.649 97.825) (end 166.263 97.439) (width 0.6) (layer "B.Cu") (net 3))
 (segment (start 166.263 97.439) (end 165.115 97.439) (width 0.6) (layer "B.Cu") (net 3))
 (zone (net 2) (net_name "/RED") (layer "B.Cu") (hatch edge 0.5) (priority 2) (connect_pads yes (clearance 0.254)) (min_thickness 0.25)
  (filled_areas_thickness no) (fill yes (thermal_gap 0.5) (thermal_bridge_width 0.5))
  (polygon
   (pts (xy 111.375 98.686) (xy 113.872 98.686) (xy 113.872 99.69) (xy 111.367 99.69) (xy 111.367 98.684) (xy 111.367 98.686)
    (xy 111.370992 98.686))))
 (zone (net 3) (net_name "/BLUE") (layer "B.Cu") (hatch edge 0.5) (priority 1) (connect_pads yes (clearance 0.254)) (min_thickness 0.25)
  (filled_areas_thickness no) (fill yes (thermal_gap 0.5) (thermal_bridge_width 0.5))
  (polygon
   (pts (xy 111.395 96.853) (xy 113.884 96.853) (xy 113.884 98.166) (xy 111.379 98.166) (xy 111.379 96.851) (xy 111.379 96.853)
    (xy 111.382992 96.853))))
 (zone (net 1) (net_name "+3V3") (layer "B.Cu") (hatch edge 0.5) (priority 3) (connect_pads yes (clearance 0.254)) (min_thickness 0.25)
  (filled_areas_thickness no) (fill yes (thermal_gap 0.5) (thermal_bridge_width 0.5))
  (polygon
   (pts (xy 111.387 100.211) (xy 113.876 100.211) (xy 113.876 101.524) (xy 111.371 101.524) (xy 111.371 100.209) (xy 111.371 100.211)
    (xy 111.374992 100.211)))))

